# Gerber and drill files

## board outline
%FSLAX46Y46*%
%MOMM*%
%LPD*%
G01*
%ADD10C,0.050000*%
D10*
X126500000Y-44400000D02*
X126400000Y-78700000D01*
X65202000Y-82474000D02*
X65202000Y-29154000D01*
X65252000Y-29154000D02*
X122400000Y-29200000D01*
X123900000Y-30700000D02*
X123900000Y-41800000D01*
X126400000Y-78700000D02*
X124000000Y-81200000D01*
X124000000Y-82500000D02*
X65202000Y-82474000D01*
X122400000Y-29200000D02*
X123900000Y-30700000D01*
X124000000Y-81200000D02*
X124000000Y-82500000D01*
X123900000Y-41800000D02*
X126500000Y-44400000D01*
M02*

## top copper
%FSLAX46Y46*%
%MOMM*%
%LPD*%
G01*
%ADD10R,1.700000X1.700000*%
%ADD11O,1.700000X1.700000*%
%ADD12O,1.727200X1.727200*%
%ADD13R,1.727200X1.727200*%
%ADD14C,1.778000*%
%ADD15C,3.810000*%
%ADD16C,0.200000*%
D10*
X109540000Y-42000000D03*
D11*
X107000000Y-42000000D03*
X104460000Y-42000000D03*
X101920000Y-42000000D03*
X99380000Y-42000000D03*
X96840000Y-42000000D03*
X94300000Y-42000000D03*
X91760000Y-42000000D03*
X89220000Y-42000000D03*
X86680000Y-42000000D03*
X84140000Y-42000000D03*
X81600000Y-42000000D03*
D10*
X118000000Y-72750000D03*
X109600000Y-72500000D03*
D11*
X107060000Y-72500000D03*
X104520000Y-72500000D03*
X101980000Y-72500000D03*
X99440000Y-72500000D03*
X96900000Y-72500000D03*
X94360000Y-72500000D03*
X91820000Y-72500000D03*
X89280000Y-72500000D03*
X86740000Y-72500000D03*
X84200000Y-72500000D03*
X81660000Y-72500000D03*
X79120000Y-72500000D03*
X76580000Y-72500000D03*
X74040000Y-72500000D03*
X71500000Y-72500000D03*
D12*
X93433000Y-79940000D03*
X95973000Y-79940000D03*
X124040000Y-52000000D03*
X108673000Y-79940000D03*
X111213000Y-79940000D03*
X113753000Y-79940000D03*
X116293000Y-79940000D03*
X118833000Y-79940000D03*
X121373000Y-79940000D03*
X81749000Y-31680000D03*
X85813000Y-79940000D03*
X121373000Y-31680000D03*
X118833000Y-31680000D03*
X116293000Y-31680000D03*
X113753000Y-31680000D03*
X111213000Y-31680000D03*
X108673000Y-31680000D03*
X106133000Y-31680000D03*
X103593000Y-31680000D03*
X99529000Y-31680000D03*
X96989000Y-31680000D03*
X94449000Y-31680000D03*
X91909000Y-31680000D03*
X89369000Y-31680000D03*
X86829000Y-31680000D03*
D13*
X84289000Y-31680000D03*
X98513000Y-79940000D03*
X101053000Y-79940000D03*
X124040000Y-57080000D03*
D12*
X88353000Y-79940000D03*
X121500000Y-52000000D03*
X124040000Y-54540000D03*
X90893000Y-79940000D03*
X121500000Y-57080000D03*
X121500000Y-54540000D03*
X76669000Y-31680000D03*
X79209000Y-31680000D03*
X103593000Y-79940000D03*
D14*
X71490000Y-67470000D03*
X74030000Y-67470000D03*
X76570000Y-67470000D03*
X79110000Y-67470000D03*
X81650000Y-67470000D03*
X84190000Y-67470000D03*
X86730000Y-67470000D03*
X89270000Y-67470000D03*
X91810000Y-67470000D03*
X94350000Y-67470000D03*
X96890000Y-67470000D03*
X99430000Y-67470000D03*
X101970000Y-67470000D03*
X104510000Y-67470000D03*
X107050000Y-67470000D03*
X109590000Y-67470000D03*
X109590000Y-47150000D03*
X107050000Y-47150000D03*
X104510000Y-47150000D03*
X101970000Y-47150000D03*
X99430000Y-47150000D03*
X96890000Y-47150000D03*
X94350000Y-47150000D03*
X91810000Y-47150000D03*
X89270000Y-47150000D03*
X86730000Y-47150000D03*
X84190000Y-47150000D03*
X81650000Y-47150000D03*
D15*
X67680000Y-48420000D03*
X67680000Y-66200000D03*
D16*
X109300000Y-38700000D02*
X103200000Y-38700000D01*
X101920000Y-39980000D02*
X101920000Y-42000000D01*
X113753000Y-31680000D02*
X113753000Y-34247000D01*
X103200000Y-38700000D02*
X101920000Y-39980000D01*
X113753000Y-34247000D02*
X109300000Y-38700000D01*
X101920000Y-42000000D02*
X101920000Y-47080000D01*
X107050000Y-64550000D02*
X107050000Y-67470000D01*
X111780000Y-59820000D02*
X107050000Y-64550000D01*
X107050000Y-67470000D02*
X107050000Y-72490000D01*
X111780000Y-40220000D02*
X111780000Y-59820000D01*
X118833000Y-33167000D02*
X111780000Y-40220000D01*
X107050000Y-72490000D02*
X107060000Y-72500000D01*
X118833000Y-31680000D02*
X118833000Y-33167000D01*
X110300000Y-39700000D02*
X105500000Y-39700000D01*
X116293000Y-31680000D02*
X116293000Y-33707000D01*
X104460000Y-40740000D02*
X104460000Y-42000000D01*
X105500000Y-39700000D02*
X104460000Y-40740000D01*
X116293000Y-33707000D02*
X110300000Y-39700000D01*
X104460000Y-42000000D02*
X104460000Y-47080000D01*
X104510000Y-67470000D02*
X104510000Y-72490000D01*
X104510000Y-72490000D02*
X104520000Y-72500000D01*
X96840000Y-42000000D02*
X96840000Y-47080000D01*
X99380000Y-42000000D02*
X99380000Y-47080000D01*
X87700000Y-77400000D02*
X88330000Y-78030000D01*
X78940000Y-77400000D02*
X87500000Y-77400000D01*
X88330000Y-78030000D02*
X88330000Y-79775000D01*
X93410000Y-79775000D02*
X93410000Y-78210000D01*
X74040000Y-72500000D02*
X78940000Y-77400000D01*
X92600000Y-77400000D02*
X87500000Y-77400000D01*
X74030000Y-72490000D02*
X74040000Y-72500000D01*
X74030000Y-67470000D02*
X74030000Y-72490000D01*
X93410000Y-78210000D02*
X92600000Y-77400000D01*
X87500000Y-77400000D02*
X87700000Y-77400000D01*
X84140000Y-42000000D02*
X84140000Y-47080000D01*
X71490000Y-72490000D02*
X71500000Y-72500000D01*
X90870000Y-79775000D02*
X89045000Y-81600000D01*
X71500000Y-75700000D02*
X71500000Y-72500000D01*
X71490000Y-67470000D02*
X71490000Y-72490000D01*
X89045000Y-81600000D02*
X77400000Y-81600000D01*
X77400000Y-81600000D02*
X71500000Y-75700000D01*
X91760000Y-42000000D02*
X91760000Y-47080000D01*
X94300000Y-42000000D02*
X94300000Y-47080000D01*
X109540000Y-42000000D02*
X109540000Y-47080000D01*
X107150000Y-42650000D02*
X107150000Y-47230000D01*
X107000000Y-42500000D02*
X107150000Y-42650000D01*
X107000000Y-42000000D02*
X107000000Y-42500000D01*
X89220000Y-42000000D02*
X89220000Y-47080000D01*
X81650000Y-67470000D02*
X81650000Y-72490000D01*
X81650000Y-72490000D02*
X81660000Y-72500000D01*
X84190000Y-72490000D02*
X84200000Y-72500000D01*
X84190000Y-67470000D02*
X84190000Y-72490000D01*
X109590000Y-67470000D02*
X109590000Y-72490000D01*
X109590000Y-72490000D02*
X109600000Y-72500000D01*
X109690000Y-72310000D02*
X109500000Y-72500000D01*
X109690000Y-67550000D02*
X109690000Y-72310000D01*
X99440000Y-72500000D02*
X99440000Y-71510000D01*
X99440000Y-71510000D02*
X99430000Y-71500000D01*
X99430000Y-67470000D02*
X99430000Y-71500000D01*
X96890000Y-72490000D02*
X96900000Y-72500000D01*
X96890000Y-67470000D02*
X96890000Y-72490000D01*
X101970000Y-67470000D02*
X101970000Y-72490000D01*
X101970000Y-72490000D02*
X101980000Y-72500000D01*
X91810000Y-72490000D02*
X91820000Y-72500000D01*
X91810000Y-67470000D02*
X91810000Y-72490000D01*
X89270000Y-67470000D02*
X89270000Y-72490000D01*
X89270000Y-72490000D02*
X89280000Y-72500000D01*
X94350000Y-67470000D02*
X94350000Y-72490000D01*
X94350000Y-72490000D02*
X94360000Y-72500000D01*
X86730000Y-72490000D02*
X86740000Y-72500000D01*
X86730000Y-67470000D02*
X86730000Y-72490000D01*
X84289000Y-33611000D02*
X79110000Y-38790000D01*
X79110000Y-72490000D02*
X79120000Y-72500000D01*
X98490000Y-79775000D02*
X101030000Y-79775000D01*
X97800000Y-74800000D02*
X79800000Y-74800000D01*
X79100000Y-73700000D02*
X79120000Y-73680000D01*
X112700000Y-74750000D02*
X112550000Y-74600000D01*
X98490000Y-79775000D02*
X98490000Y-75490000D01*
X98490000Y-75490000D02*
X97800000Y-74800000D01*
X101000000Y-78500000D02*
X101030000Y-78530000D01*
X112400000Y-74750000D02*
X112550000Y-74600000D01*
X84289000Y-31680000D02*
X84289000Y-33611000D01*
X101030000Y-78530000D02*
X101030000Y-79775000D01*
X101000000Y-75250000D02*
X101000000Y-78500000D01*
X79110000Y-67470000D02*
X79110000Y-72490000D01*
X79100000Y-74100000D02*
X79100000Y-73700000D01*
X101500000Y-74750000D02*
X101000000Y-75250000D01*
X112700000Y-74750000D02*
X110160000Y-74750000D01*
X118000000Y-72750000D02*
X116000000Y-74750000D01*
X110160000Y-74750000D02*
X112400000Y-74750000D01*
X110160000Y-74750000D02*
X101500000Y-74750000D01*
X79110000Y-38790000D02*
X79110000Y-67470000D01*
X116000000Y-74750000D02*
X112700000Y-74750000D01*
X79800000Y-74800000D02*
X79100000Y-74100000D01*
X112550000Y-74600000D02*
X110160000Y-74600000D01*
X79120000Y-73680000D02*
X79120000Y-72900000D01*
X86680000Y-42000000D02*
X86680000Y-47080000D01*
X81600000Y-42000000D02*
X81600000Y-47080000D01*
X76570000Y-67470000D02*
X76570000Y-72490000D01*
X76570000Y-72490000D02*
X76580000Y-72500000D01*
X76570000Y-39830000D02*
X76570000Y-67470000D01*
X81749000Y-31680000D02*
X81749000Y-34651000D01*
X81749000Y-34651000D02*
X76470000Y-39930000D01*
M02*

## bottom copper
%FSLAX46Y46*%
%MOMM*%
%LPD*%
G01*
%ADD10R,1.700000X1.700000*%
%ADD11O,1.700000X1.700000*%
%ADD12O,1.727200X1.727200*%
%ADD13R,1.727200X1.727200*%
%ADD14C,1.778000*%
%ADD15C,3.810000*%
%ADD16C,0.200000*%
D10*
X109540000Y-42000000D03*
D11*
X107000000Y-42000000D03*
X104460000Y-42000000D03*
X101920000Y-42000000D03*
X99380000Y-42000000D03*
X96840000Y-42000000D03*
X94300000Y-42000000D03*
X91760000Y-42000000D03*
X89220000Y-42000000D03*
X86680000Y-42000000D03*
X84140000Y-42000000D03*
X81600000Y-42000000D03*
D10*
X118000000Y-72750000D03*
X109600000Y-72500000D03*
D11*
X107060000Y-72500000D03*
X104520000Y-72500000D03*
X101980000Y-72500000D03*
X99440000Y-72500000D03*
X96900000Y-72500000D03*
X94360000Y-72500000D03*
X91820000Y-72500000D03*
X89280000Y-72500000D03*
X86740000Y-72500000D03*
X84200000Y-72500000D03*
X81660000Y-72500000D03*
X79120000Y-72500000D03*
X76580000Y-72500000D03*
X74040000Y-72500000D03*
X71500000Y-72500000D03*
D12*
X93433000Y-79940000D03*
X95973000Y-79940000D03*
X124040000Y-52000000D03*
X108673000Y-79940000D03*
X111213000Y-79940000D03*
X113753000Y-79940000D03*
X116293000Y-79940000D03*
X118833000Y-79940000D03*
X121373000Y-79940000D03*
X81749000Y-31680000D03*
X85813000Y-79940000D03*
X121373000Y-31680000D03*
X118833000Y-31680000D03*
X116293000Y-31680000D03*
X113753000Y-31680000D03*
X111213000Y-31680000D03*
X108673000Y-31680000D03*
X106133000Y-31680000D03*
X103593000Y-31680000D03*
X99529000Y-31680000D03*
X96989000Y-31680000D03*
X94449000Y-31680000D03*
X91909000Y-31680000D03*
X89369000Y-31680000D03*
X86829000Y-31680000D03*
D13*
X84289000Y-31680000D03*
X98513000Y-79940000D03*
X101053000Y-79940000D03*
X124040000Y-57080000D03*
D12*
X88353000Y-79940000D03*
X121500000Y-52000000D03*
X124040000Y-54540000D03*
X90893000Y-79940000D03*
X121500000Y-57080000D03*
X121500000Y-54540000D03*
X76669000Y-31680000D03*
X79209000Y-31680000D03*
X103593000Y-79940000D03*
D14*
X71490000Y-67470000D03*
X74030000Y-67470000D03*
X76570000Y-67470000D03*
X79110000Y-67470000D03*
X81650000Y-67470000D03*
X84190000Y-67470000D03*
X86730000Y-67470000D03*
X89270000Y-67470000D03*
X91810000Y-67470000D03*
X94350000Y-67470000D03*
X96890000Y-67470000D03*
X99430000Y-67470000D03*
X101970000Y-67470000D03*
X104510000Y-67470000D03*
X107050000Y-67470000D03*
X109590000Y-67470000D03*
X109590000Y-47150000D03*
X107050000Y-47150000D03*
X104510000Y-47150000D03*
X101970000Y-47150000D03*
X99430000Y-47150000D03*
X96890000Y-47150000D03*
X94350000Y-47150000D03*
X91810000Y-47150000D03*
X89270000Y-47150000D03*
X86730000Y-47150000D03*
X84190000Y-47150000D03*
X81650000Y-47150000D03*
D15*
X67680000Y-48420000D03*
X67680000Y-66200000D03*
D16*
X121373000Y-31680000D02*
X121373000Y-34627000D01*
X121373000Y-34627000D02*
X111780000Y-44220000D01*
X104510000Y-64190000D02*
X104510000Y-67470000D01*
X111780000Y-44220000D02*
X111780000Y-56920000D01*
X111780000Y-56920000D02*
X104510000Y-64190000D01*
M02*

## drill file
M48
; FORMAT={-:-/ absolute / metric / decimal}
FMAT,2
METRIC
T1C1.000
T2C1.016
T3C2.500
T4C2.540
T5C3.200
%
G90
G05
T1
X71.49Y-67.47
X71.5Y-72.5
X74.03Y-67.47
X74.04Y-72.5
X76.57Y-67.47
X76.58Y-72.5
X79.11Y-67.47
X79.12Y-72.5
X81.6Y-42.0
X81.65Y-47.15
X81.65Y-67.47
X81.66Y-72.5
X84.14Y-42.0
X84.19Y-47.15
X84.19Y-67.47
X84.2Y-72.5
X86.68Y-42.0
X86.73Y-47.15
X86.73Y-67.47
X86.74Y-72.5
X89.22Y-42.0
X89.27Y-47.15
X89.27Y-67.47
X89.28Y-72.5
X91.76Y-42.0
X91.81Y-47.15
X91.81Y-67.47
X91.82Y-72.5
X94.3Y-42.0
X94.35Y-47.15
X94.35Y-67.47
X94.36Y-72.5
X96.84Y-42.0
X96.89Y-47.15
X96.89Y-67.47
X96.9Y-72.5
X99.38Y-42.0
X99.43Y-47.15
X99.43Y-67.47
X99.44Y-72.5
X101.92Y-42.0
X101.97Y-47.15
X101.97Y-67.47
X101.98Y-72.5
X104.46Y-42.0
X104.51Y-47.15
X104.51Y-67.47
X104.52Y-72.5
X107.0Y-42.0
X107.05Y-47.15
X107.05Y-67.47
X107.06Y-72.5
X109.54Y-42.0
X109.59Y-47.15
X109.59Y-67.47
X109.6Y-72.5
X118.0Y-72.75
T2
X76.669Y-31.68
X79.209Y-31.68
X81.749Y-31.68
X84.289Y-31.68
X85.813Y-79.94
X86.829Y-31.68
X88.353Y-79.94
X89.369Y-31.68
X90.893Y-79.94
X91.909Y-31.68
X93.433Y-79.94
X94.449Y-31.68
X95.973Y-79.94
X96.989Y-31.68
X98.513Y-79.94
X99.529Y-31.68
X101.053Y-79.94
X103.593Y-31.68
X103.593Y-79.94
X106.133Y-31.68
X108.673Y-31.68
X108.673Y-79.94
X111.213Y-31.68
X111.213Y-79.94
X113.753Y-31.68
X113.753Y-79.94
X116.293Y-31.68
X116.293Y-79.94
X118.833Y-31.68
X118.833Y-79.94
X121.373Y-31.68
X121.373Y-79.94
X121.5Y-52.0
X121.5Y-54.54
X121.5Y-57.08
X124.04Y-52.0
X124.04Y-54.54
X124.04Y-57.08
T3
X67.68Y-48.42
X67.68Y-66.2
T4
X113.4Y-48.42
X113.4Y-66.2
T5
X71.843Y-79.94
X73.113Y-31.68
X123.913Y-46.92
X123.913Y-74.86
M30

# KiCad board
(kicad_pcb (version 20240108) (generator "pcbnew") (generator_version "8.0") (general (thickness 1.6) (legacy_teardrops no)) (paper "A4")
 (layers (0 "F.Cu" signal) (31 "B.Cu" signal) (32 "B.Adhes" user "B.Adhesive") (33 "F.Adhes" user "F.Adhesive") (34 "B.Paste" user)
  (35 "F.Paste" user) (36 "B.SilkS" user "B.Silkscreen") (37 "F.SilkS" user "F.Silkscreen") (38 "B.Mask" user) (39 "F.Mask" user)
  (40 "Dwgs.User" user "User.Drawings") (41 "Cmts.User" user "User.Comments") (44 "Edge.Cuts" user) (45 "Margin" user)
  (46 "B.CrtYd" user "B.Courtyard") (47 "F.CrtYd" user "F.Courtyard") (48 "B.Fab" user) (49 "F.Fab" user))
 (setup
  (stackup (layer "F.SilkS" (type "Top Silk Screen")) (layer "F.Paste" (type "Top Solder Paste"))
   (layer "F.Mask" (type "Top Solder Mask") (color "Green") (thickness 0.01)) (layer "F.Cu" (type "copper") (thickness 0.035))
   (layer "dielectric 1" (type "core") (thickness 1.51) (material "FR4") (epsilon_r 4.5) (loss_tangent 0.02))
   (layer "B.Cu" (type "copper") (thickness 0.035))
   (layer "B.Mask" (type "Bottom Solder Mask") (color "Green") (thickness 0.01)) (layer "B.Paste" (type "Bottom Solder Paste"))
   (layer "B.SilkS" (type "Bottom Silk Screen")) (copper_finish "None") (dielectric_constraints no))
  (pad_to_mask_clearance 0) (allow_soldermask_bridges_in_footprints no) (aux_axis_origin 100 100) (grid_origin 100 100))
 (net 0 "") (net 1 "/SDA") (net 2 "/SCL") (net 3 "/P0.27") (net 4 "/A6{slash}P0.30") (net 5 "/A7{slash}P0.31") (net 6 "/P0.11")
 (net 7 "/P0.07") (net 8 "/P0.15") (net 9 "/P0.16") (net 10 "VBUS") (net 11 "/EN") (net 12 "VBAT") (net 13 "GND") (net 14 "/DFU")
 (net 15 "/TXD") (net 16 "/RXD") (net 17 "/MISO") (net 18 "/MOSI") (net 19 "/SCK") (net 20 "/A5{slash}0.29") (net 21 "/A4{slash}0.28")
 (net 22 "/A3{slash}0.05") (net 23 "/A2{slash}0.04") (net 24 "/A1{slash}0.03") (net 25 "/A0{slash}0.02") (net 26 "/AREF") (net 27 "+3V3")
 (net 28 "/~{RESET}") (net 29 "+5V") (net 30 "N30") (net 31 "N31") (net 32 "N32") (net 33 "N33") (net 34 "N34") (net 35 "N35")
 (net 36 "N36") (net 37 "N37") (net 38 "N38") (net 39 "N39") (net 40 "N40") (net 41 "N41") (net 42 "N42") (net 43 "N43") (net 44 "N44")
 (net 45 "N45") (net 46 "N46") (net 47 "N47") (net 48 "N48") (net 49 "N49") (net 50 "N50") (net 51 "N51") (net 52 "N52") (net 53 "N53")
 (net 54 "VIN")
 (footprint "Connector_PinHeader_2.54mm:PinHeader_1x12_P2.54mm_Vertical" (layer "F.Cu") (at 109.54 42 -90)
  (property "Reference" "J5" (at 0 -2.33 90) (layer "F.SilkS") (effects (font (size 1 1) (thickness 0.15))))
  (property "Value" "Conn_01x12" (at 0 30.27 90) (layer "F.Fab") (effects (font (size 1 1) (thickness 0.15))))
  (pad "1" thru_hole rect (at 0 0 270) (size 1.7 1.7) (drill 1) (layers "*.Cu" "*.Mask") (remove_unused_layers no) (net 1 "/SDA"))
  (pad "2" thru_hole oval (at 0 2.54 270) (size 1.7 1.7) (drill 1) (layers "*.Cu" "*.Mask") (remove_unused_layers no) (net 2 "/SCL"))
  (pad "3" thru_hole oval (at 0 5.08 270) (size 1.7 1.7) (drill 1) (layers "*.Cu" "*.Mask") (remove_unused_layers no) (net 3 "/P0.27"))
  (pad "4" thru_hole oval (at 0 7.62 270) (size 1.7 1.7) (drill 1) (layers "*.Cu" "*.Mask") (remove_unused_layers no)
   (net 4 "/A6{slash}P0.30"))
  (pad "5" thru_hole oval (at 0 10.16 270) (size 1.7 1.7) (drill 1) (layers "*.Cu" "*.Mask") (remove_unused_layers no)
   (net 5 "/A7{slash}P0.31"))
  (pad "6" thru_hole oval (at 0 12.7 270) (size 1.7 1.7) (drill 1) (layers "*.Cu" "*.Mask") (remove_unused_layers no) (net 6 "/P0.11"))
  (pad "7" thru_hole oval (at 0 15.24 270) (size 1.7 1.7) (drill 1) (layers "*.Cu" "*.Mask") (remove_unused_layers no) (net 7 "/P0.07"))
  (pad "8" thru_hole oval (at 0 17.78 270) (size 1.7 1.7) (drill 1) (layers "*.Cu" "*.Mask") (remove_unused_layers no) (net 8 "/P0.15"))
  (pad "9" thru_hole oval (at 0 20.32 270) (size 1.7 1.7) (drill 1) (layers "*.Cu" "*.Mask") (remove_unused_layers no) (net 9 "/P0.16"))
  (pad "10" thru_hole oval (at 0 22.86 270) (size 1.7 1.7) (drill 1) (layers "*.Cu" "*.Mask") (remove_unused_layers no) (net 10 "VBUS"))
  (pad "11" thru_hole oval (at 0 25.4 270) (size 1.7 1.7) (drill 1) (layers "*.Cu" "*.Mask") (remove_unused_layers no) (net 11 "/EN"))
  (pad "12" thru_hole oval (at 0 27.94 270) (size 1.7 1.7) (drill 1) (layers "*.Cu" "*.Mask") (remove_unused_layers no) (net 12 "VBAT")))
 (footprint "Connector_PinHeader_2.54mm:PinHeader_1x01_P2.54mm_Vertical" (layer "F.Cu") (at 118 72.75)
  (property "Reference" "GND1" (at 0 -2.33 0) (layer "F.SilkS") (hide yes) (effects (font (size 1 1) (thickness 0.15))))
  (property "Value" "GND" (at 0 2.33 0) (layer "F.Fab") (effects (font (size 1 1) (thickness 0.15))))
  (pad "1" thru_hole rect (at 0 0) (size 1.7 1.7) (drill 1) (layers "*.Cu" "*.Mask") (remove_unused_layers no) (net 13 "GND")))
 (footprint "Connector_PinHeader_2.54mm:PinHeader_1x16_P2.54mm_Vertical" (layer "F.Cu") (at 109.6 72.5 -90)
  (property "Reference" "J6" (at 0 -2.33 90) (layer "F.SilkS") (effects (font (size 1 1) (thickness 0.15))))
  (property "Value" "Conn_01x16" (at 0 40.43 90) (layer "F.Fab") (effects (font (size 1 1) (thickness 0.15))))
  (pad "1" thru_hole rect (at 0 0 270) (size 1.7 1.7) (drill 1) (layers "*.Cu" "*.Mask") (remove_unused_layers no) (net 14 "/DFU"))
  (pad "2" thru_hole oval (at 0 2.54 270) (size 1.7 1.7) (drill 1) (layers "*.Cu" "*.Mask") (remove_unused_layers no) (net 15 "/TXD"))
  (pad "3" thru_hole oval (at 0 5.08 270) (size 1.7 1.7) (drill 1) (layers "*.Cu" "*.Mask") (remove_unused_layers no) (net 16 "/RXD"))
  (pad "4" thru_hole oval (at 0 7.62 270) (size 1.7 1.7) (drill 1) (layers "*.Cu" "*.Mask") (remove_unused_layers no) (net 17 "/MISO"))
  (pad "5" thru_hole oval (at 0 10.16 270) (size 1.7 1.7) (drill 1) (layers "*.Cu" "*.Mask") (remove_unused_layers no) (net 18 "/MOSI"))
  (pad "6" thru_hole oval (at 0 12.7 270) (size 1.7 1.7) (drill 1) (layers "*.Cu" "*.Mask") (remove_unused_layers no) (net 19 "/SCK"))
  (pad "7" thru_hole oval (at 0 15.24 270) (size 1.7 1.7) (drill 1) (layers "*.Cu" "*.Mask") (remove_unused_layers no)
   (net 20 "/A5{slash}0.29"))
  (pad "8" thru_hole oval (at 0 17.78 270) (size 1.7 1.7) (drill 1) (layers "*.Cu" "*.Mask") (remove_unused_layers no)
   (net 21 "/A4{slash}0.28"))
  (pad "9" thru_hole oval (at 0 20.32 270) (size 1.7 1.7) (drill 1) (layers "*.Cu" "*.Mask") (remove_unused_layers no)
   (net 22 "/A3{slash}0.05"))
  (pad "10" thru_hole oval (at 0 22.86 270) (size 1.7 1.7) (drill 1) (layers "*.Cu" "*.Mask") (remove_unused_layers no)
   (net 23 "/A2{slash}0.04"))
  (pad "11" thru_hole oval (at 0 25.4 270) (size 1.7 1.7) (drill 1) (layers "*.Cu" "*.Mask") (remove_unused_layers no)
   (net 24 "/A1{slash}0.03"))
  (pad "12" thru_hole oval (at 0 27.94 270) (size 1.7 1.7) (drill 1) (layers "*.Cu" "*.Mask") (remove_unused_layers no)
   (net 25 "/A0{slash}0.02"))
  (pad "13" thru_hole oval (at 0 30.48 270) (size 1.7 1.7) (drill 1) (layers "*.Cu" "*.Mask") (remove_unused_layers no) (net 13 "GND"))
  (pad "14" thru_hole oval (at 0 33.02 270) (size 1.7 1.7) (drill 1) (layers "*.Cu" "*.Mask") (remove_unused_layers no) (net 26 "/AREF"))
  (pad "15" thru_hole oval (at 0 35.56 270) (size 1.7 1.7) (drill 1) (layers "*.Cu" "*.Mask") (remove_unused_layers no) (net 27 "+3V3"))
  (pad "16" thru_hole oval (at 0 38.1 270) (size 1.7 1.7) (drill 1) (layers "*.Cu" "*.Mask") (remove_unused_layers no) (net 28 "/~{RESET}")))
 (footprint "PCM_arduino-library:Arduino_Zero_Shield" (layer "F.Cu") (at 57.873 82.48)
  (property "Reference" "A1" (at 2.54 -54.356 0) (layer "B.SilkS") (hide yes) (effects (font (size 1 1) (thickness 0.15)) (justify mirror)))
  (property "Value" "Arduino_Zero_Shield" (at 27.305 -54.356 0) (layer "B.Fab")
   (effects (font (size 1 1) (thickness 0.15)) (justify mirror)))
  (pad "" np_thru_hole circle (at 13.97 -2.54) (size 3.2 3.2) (drill 3.2) (layers "*.Cu" "*.Mask"))
  (pad "" np_thru_hole circle (at 15.24 -50.8) (size 3.2 3.2) (drill 3.2) (layers "*.Cu" "*.Mask"))
  (pad "" np_thru_hole circle (at 66.04 -35.56) (size 3.2 3.2) (drill 3.2) (layers "*.Cu" "*.Mask"))
  (pad "" np_thru_hole circle (at 66.04 -7.62) (size 3.2 3.2) (drill 3.2) (layers "*.Cu" "*.Mask"))
  (pad "3V3" thru_hole oval (at 35.56 -2.54) (size 1.7272 1.7272) (drill 1.016) (layers "*.Cu" "*.Mask") (remove_unused_layers no)
   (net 27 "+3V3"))
  (pad "5V1" thru_hole oval (at 38.1 -2.54) (size 1.7272 1.7272) (drill 1.016) (layers "*.Cu" "*.Mask") (remove_unused_layers no)
   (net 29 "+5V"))
  (pad "5V2" thru_hole oval (at 66.167 -30.48) (size 1.7272 1.7272) (drill 1.016) (layers "*.Cu" "*.Mask") (remove_unused_layers no)
   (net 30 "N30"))
  (pad "A0" thru_hole oval (at 50.8 -2.54) (size 1.7272 1.7272) (drill 1.016) (layers "*.Cu" "*.Mask") (remove_unused_layers no)
   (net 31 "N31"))
  (pad "A1" thru_hole oval (at 53.34 -2.54) (size 1.7272 1.7272) (drill 1.016) (layers "*.Cu" "*.Mask") (remove_unused_layers no)
   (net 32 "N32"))
  (pad "A2" thru_hole oval (at 55.88 -2.54) (size 1.7272 1.7272) (drill 1.016) (layers "*.Cu" "*.Mask") (remove_unused_layers no)
   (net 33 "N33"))
  (pad "A3" thru_hole oval (at 58.42 -2.54) (size 1.7272 1.7272) (drill 1.016) (layers "*.Cu" "*.Mask") (remove_unused_layers no)
   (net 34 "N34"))
  (pad "A4" thru_hole oval (at 60.96 -2.54) (size 1.7272 1.7272) (drill 1.016) (layers "*.Cu" "*.Mask") (remove_unused_layers no)
   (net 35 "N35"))
  (pad "A5" thru_hole oval (at 63.5 -2.54) (size 1.7272 1.7272) (drill 1.016) (layers "*.Cu" "*.Mask") (remove_unused_layers no)
   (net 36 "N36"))
  (pad "AREF" thru_hole oval (at 23.876 -50.8) (size 1.7272 1.7272) (drill 1.016) (layers "*.Cu" "*.Mask") (remove_unused_layers no)
   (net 26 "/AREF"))
  (pad "ATN" thru_hole oval (at 27.94 -2.54) (size 1.7272 1.7272) (drill 1.016) (layers "*.Cu" "*.Mask") (remove_unused_layers no)
   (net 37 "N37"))
  (pad "D0" thru_hole oval (at 63.5 -50.8) (size 1.7272 1.7272) (drill 1.016) (layers "*.Cu" "*.Mask") (remove_unused_layers no)
   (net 16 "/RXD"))
  (pad "D1" thru_hole oval (at 60.96 -50.8) (size 1.7272 1.7272) (drill 1.016) (layers "*.Cu" "*.Mask") (remove_unused_layers no)
   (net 15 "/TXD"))
  (pad "D2" thru_hole oval (at 58.42 -50.8) (size 1.7272 1.7272) (drill 1.016) (layers "*.Cu" "*.Mask") (remove_unused_layers no)
   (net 3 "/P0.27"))
  (pad "D3" thru_hole oval (at 55.88 -50.8) (size 1.7272 1.7272) (drill 1.016) (layers "*.Cu" "*.Mask") (remove_unused_layers no)
   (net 4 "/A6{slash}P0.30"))
  (pad "D4" thru_hole oval (at 53.34 -50.8) (size 1.7272 1.7272) (drill 1.016) (layers "*.Cu" "*.Mask") (remove_unused_layers no)
   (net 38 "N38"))
  (pad "D5" thru_hole oval (at 50.8 -50.8) (size 1.7272 1.7272) (drill 1.016) (layers "*.Cu" "*.Mask") (remove_unused_layers no)
   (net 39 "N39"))
  (pad "D6" thru_hole oval (at 48.26 -50.8) (size 1.7272 1.7272) (drill 1.016) (layers "*.Cu" "*.Mask") (remove_unused_layers no)
   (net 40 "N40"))
  (pad "D7" thru_hole oval (at 45.72 -50.8) (size 1.7272 1.7272) (drill 1.016) (layers "*.Cu" "*.Mask") (remove_unused_layers no)
   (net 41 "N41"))
  (pad "D8" thru_hole oval (at 41.656 -50.8) (size 1.7272 1.7272) (drill 1.016) (layers "*.Cu" "*.Mask") (remove_unused_layers no)
   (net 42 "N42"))
  (pad "D9" thru_hole oval (at 39.116 -50.8) (size 1.7272 1.7272) (drill 1.016) (layers "*.Cu" "*.Mask") (remove_unused_layers no)
   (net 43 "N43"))
  (pad "D10" thru_hole oval (at 36.576 -50.8) (size 1.7272 1.7272) (drill 1.016) (layers "*.Cu" "*.Mask") (remove_unused_layers no)
   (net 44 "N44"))
  (pad "D11" thru_hole oval (at 34.036 -50.8) (size 1.7272 1.7272) (drill 1.016) (layers "*.Cu" "*.Mask") (remove_unused_layers no)
   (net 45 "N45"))
  (pad "D12" thru_hole oval (at 31.496 -50.8) (size 1.7272 1.7272) (drill 1.016) (layers "*.Cu" "*.Mask") (remove_unused_layers no)
   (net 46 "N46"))
  (pad "D13" thru_hole oval (at 28.956 -50.8) (size 1.7272 1.7272) (drill 1.016) (layers "*.Cu" "*.Mask") (remove_unused_layers no)
   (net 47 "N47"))
  (pad "GND1" thru_hole rect (at 26.416 -50.8) (size 1.7272 1.7272) (drill 1.016) (layers "*.Cu" "*.Mask") (remove_unused_layers no)
   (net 13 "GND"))
  (pad "GND2" thru_hole rect (at 40.64 -2.54) (size 1.7272 1.7272) (drill 1.016) (layers "*.Cu" "*.Mask") (remove_unused_layers no)
   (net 13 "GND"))
  (pad "GND3" thru_hole rect (at 43.18 -2.54) (size 1.7272 1.7272) (drill 1.016) (layers "*.Cu" "*.Mask") (remove_unused_layers no)
   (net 13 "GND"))
  (pad "GND4" thru_hole rect (at 66.167 -25.4) (size 1.7272 1.7272) (drill 1.016) (layers "*.Cu" "*.Mask") (remove_unused_layers no)
   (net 13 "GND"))
  (pad "IORF" thru_hole oval (at 30.48 -2.54) (size 1.7272 1.7272) (drill 1.016) (layers "*.Cu" "*.Mask") (remove_unused_layers no)
   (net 27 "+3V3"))
  (pad "MISO" thru_hole oval (at 63.627 -30.48) (size 1.7272 1.7272) (drill 1.016) (layers "*.Cu" "*.Mask") (remove_unused_layers no)
   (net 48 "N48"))
  (pad "MOSI" thru_hole oval (at 66.167 -27.94) (size 1.7272 1.7272) (drill 1.016) (layers "*.Cu" "*.Mask") (remove_unused_layers no)
   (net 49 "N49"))
  (pad "RST1" thru_hole oval (at 33.02 -2.54) (size 1.7272 1.7272) (drill 1.016) (layers "*.Cu" "*.Mask") (remove_unused_layers no)
   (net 28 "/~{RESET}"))
  (pad "RST2" thru_hole oval (at 63.627 -25.4) (size 1.7272 1.7272) (drill 1.016) (layers "*.Cu" "*.Mask") (remove_unused_layers no)
   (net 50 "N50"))
  (pad "SCK" thru_hole oval (at 63.627 -27.94) (size 1.7272 1.7272) (drill 1.016) (layers "*.Cu" "*.Mask") (remove_unused_layers no)
   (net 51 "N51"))
  (pad "SCL" thru_hole oval (at 18.796 -50.8) (size 1.7272 1.7272) (drill 1.016) (layers "*.Cu" "*.Mask") (remove_unused_layers no)
   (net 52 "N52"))
  (pad "SDA" thru_hole oval (at 21.336 -50.8) (size 1.7272 1.7272) (drill 1.016) (layers "*.Cu" "*.Mask") (remove_unused_layers no)
   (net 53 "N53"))
  (pad "VIN" thru_hole oval (at 45.72 -2.54) (size 1.7272 1.7272) (drill 1.016) (layers "*.Cu" "*.Mask") (remove_unused_layers no)
   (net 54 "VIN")))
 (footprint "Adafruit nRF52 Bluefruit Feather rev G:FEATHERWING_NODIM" (layer "F.Cu") (at 65.14 68.74)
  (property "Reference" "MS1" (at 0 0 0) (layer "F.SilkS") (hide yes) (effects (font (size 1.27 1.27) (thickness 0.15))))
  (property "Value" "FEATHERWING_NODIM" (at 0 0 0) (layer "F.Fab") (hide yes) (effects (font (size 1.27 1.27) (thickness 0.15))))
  (pad "" np_thru_hole circle (at 48.26 -20.32) (size 2.54 2.54) (drill 2.54) (layers "*.Cu" "*.Mask"))
  (pad "" np_thru_hole circle (at 48.26 -2.54) (size 2.54 2.54) (drill 2.54) (layers "*.Cu" "*.Mask"))
  (pad "1" thru_hole circle (at 6.35 -1.27) (size 1.778 1.778) (drill 1) (layers "*.Cu" "*.Mask") (remove_unused_layers no)
   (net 28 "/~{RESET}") (solder_mask_margin 0.0508) (thermal_bridge_angle 0))
  (pad "2" thru_hole circle (at 8.89 -1.27) (size 1.778 1.778) (drill 1) (layers "*.Cu" "*.Mask") (remove_unused_layers no) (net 27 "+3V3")
   (solder_mask_margin 0.0508) (thermal_bridge_angle 0))
  (pad "3" thru_hole circle (at 11.43 -1.27) (size 1.778 1.778) (drill 1) (layers "*.Cu" "*.Mask") (remove_unused_layers no)
   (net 26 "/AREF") (solder_mask_margin 0.0508) (thermal_bridge_angle 0))
  (pad "4" thru_hole circle (at 13.97 -1.27) (size 1.778 1.778) (drill 1) (layers "*.Cu" "*.Mask") (remove_unused_layers no) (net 13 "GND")
   (solder_mask_margin 0.0508) (thermal_bridge_angle 0))
  (pad "5" thru_hole circle (at 16.51 -1.27) (size 1.778 1.778) (drill 1) (layers "*.Cu" "*.Mask") (remove_unused_layers no)
   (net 25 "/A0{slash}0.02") (solder_mask_margin 0.0508) (thermal_bridge_angle 0))
  (pad "6" thru_hole circle (at 19.05 -1.27) (size 1.778 1.778) (drill 1) (layers "*.Cu" "*.Mask") (remove_unused_layers no)
   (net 24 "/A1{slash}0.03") (solder_mask_margin 0.0508) (thermal_bridge_angle 0))
  (pad "7" thru_hole circle (at 21.59 -1.27) (size 1.778 1.778) (drill 1) (layers "*.Cu" "*.Mask") (remove_unused_layers no)
   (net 23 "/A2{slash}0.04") (solder_mask_margin 0.0508) (thermal_bridge_angle 0))
  (pad "8" thru_hole circle (at 24.13 -1.27) (size 1.778 1.778) (drill 1) (layers "*.Cu" "*.Mask") (remove_unused_layers no)
   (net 22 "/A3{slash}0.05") (solder_mask_margin 0.0508) (thermal_bridge_angle 0))
  (pad "9" thru_hole circle (at 26.67 -1.27) (size 1.778 1.778) (drill 1) (layers "*.Cu" "*.Mask") (remove_unused_layers no)
   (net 21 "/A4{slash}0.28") (solder_mask_margin 0.0508) (thermal_bridge_angle 0))
  (pad "10" thru_hole circle (at 29.21 -1.27) (size 1.778 1.778) (drill 1) (layers "*.Cu" "*.Mask") (remove_unused_layers no)
   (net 20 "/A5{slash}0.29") (solder_mask_margin 0.0508) (thermal_bridge_angle 0))
  (pad "11" thru_hole circle (at 31.75 -1.27) (size 1.778 1.778) (drill 1) (layers "*.Cu" "*.Mask") (remove_unused_layers no)
   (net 19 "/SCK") (solder_mask_margin 0.0508) (thermal_bridge_angle 0))
  (pad "12" thru_hole circle (at 34.29 -1.27) (size 1.778 1.778) (drill 1) (layers "*.Cu" "*.Mask") (remove_unused_layers no)
   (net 18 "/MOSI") (solder_mask_margin 0.0508) (thermal_bridge_angle 0))
  (pad "13" thru_hole circle (at 36.83 -1.27) (size 1.778 1.778) (drill 1) (layers "*.Cu" "*.Mask") (remove_unused_layers no)
   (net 17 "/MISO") (solder_mask_margin 0.0508) (thermal_bridge_angle 0))
  (pad "14" thru_hole circle (at 39.37 -1.27) (size 1.778 1.778) (drill 1) (layers "*.Cu" "*.Mask") (remove_unused_layers no)
   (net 16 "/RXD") (solder_mask_margin 0.0508) (thermal_bridge_angle 0))
  (pad "15" thru_hole circle (at 41.91 -1.27) (size 1.778 1.778) (drill 1) (layers "*.Cu" "*.Mask") (remove_unused_layers no)
   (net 15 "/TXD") (solder_mask_margin 0.0508) (thermal_bridge_angle 0))
  (pad "16" thru_hole circle (at 44.45 -1.27) (size 1.778 1.778) (drill 1) (layers "*.Cu" "*.Mask") (remove_unused_layers no)
   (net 14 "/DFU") (solder_mask_margin 0.0508) (thermal_bridge_angle 0))
  (pad "17" thru_hole circle (at 44.45 -21.59) (size 1.778 1.778) (drill 1) (layers "*.Cu" "*.Mask") (remove_unused_layers no)
   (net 1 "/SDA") (solder_mask_margin 0.0508) (thermal_bridge_angle 0))
  (pad "18" thru_hole circle (at 41.91 -21.59) (size 1.778 1.778) (drill 1) (layers "*.Cu" "*.Mask") (remove_unused_layers no)
   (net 2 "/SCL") (solder_mask_margin 0.0508) (thermal_bridge_angle 0))
  (pad "19" thru_hole circle (at 39.37 -21.59) (size 1.778 1.778) (drill 1) (layers "*.Cu" "*.Mask") (remove_unused_layers no)
   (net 3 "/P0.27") (solder_mask_margin 0.0508) (thermal_bridge_angle 0))
  (pad "20" thru_hole circle (at 36.83 -21.59) (size 1.778 1.778) (drill 1) (layers "*.Cu" "*.Mask") (remove_unused_layers no)
   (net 4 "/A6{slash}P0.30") (solder_mask_margin 0.0508) (thermal_bridge_angle 0))
  (pad "21" thru_hole circle (at 34.29 -21.59) (size 1.778 1.778) (drill 1) (layers "*.Cu" "*.Mask") (remove_unused_layers no)
   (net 5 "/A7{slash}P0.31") (solder_mask_margin 0.0508) (thermal_bridge_angle 0))
  (pad "22" thru_hole circle (at 31.75 -21.59) (size 1.778 1.778) (drill 1) (layers "*.Cu" "*.Mask") (remove_unused_layers no)
   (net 6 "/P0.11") (solder_mask_margin 0.0508) (thermal_bridge_angle 0))
  (pad "23" thru_hole circle (at 29.21 -21.59) (size 1.778 1.778) (drill 1) (layers "*.Cu" "*.Mask") (remove_unused_layers no)
   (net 7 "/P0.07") (solder_mask_margin 0.0508) (thermal_bridge_angle 0))
  (pad "24" thru_hole circle (at 26.67 -21.59) (size 1.778 1.778) (drill 1) (layers "*.Cu" "*.Mask") (remove_unused_layers no)
   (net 8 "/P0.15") (solder_mask_margin 0.0508) (thermal_bridge_angle 0))
  (pad "25" thru_hole circle (at 24.13 -21.59) (size 1.778 1.778) (drill 1) (layers "*.Cu" "*.Mask") (remove_unused_layers no)
   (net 9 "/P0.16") (solder_mask_margin 0.0508) (thermal_bridge_angle 0))
  (pad "26" thru_hole circle (at 21.59 -21.59) (size 1.778 1.778) (drill 1) (layers "*.Cu" "*.Mask") (remove_unused_layers no)
   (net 10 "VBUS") (solder_mask_margin 0.0508) (thermal_bridge_angle 0))
  (pad "27" thru_hole circle (at 19.05 -21.59) (size 1.778 1.778) (drill 1) (layers "*.Cu" "*.Mask") (remove_unused_layers no)
   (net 11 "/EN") (solder_mask_margin 0.0508) (thermal_bridge_angle 0))
  (pad "28" thru_hole circle (at 16.51 -21.59) (size 1.778 1.778) (drill 1) (layers "*.Cu" "*.Mask") (remove_unused_layers no)
   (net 12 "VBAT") (solder_mask_margin 0.0508) (thermal_bridge_angle 0))
  (pad "P$1" thru_hole circle (at 2.54 -20.32) (size 3.81 3.81) (drill 2.5) (layers "*.Cu" "*.Mask") (remove_unused_layers no)
   (solder_mask_margin 0.0508) (thermal_bridge_angle 0))
  (pad "P$2" thru_hole circle (at 2.54 -2.54) (size 3.81 3.81) (drill 2.5) (layers "*.Cu" "*.Mask") (remove_unused_layers no)
   (solder_mask_margin 0.0508) (thermal_bridge_angle 0)))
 (gr_line (start 126.5 44.4) (end 126.4 78.7) (stroke (width 0.05) (type default)) (layer "Edge.Cuts"))
 (gr_line (start 65.202 82.474) (end 65.202 29.154) (stroke (width 0.05) (type default)) (layer "Edge.Cuts"))
 (gr_line (start 65.252 29.154) (end 122.4 29.2) (stroke (width 0.05) (type default)) (layer "Edge.Cuts"))
 (gr_line (start 123.9 30.7) (end 123.9 41.8) (stroke (width 0.05) (type default)) (layer "Edge.Cuts"))
 (gr_line (start 126.4 78.7) (end 124 81.2) (stroke (width 0.05) (type default)) (layer "Edge.Cuts"))
 (gr_line (start 124 82.5) (end 65.202 82.474) (stroke (width 0.05) (type default)) (layer "Edge.Cuts"))
 (gr_line (start 122.4 29.2) (end 123.9 30.7) (stroke (width 0.05) (type default)) (layer "Edge.Cuts"))
 (gr_line (start 124 81.2) (end 124 82.5) (stroke (width 0.05) (type default)) (layer "Edge.Cuts"))
 (gr_line (start 123.9 41.8) (end 126.5 44.4) (stroke (width 0.05) (type default)) (layer "Edge.Cuts"))
 (segment (start 109.3 38.7) (end 103.2 38.7) (width 0.2) (layer "F.Cu") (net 4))
 (segment (start 101.92 39.98) (end 101.92 42) (width 0.2) (layer "F.Cu") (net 4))
 (segment (start 113.753 31.68) (end 113.753 34.247) (width 0.2) (layer "F.Cu") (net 4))
 (segment (start 103.2 38.7) (end 101.92 39.98) (width 0.2) (layer "F.Cu") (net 4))
 (segment (start 113.753 34.247) (end 109.3 38.7) (width 0.2) (layer "F.Cu") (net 4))
 (segment (start 101.92 42) (end 101.92 47.08) (width 0.2) (layer "F.Cu") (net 4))
 (segment (start 107.05 64.55) (end 107.05 67.47) (width 0.2) (layer "F.Cu") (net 15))
 (segment (start 111.78 59.82) (end 107.05 64.55) (width 0.2) (layer "F.Cu") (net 15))
 (segment (start 107.05 67.47) (end 107.05 72.49) (width 0.2) (layer "F.Cu") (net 15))
 (segment (start 111.78 40.22) (end 111.78 59.82) (width 0.2) (layer "F.Cu") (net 15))
 (segment (start 118.833 33.167) (end 111.78 40.22) (width 0.2) (layer "F.Cu") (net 15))
 (segment (start 107.05 72.49) (end 107.06 72.5) (width 0.2) (layer "F.Cu") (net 15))
 (segment (start 118.833 31.68) (end 118.833 33.167) (width 0.2) (layer "F.Cu") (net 15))
 (segment (start 110.3 39.7) (end 105.5 39.7) (width 0.2) (layer "F.Cu") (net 3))
 (segment (start 116.293 31.68) (end 116.293 33.707) (width 0.2) (layer "F.Cu") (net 3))
 (segment (start 104.46 40.74) (end 104.46 42) (width 0.2) (layer "F.Cu") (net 3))
 (segment (start 105.5 39.7) (end 104.46 40.74) (width 0.2) (layer "F.Cu") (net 3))
 (segment (start 116.293 33.707) (end 110.3 39.7) (width 0.2) (layer "F.Cu") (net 3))
 (segment (start 104.46 42) (end 104.46 47.08) (width 0.2) (layer "F.Cu") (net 3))
 (segment (start 104.51 67.47) (end 104.51 72.49) (width 0.2) (layer "F.Cu") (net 16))
 (segment (start 104.51 72.49) (end 104.52 72.5) (width 0.2) (layer "F.Cu") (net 16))
 (segment (start 121.373 31.68) (end 121.373 34.627) (width 0.2) (layer "B.Cu") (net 16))
 (segment (start 121.373 34.627) (end 111.78 44.22) (width 0.2) (layer "B.Cu") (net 16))
 (segment (start 104.51 64.19) (end 104.51 67.47) (width 0.2) (layer "B.Cu") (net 16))
 (segment (start 111.78 44.22) (end 111.78 56.92) (width 0.2) (layer "B.Cu") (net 16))
 (segment (start 111.78 56.92) (end 104.51 64.19) (width 0.2) (layer "B.Cu") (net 16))
 (segment (start 96.84 42) (end 96.84 47.08) (width 0.2) (layer "F.Cu") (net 6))
 (segment (start 99.38 42) (end 99.38 47.08) (width 0.2) (layer "F.Cu") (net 5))
 (segment (start 87.7 77.4) (end 88.33 78.03) (width 0.2) (layer "F.Cu") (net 27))
 (segment (start 78.94 77.4) (end 87.5 77.4) (width 0.2) (layer "F.Cu") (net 27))
 (segment (start 88.33 78.03) (end 88.33 79.775) (width 0.2) (layer "F.Cu") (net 27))
 (segment (start 93.41 79.775) (end 93.41 78.21) (width 0.2) (layer "F.Cu") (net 27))
 (segment (start 74.04 72.5) (end 78.94 77.4) (width 0.2) (layer "F.Cu") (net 27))
 (segment (start 92.6 77.4) (end 87.5 77.4) (width 0.2) (layer "F.Cu") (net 27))
 (segment (start 74.03 72.49) (end 74.04 72.5) (width 0.2) (layer "F.Cu") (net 27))
 (segment (start 74.03 67.47) (end 74.03 72.49) (width 0.2) (layer "F.Cu") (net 27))
 (segment (start 93.41 78.21) (end 92.6 77.4) (width 0.2) (layer "F.Cu") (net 27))
 (segment (start 87.5 77.4) (end 87.7 77.4) (width 0.2) (layer "F.Cu") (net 27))
 (segment (start 84.14 42) (end 84.14 47.08) (width 0.2) (layer "F.Cu") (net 11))
 (segment (start 71.49 72.49) (end 71.5 72.5) (width 0.2) (layer "F.Cu") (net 28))
 (segment (start 90.87 79.775) (end 89.045 81.6) (width 0.2) (layer "F.Cu") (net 28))
 (segment (start 71.5 75.7) (end 71.5 72.5) (width 0.2) (layer "F.Cu") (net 28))
 (segment (start 71.49 67.47) (end 71.49 72.49) (width 0.2) (layer "F.Cu") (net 28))
 (segment (start 89.045 81.6) (end 77.4 81.6) (width 0.2) (layer "F.Cu") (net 28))
 (segment (start 77.4 81.6) (end 71.5 75.7) (width 0.2) (layer "F.Cu") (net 28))
 (segment (start 91.76 42) (end 91.76 47.08) (width 0.2) (layer "F.Cu") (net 8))
 (segment (start 94.3 42) (end 94.3 47.08) (width 0.2) (layer "F.Cu") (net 7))
 (segment (start 109.54 42) (end 109.54 47.08) (width 0.2) (layer "F.Cu") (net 1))
 (segment (start 107.15 42.65) (end 107.15 47.23) (width 0.2) (layer "F.Cu") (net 2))
 (segment (start 107 42.5) (end 107.15 42.65) (width 0.2) (layer "F.Cu") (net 2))
 (segment (start 107 42) (end 107 42.5) (width 0.2) (layer "F.Cu") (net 2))
 (segment (start 89.22 42) (end 89.22 47.08) (width 0.2) (layer "F.Cu") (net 9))
 (segment (start 81.65 67.47) (end 81.65 72.49) (width 0.2) (layer "F.Cu") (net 25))
 (segment (start 81.65 72.49) (end 81.66 72.5) (width 0.2) (layer "F.Cu") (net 25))
 (segment (start 84.19 72.49) (end 84.2 72.5) (width 0.2) (layer "F.Cu") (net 24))
 (segment (start 84.19 67.47) (end 84.19 72.49) (width 0.2) (layer "F.Cu") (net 24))
 (segment (start 109.59 67.47) (end 109.59 72.49) (width 0.2) (layer "F.Cu") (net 14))
 (segment (start 109.59 72.49) (end 109.6 72.5) (width 0.2) (layer "F.Cu") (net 14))
 (segment (start 109.69 72.31) (end 109.5 72.5) (width 0.2) (layer "F.Cu") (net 14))
 (segment (start 109.69 67.55) (end 109.69 72.31) (width 0.2) (layer "F.Cu") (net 14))
 (segment (start 99.44 72.5) (end 99.44 71.51) (width 0.2) (layer "F.Cu") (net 18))
 (segment (start 99.44 71.51) (end 99.43 71.5) (width 0.2) (layer "F.Cu") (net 18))
 (segment (start 99.43 67.47) (end 99.43 71.5) (width 0.2) (layer "F.Cu") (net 18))
 (segment (start 96.89 72.49) (end 96.9 72.5) (width 0.2) (layer "F.Cu") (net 19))
 (segment (start 96.89 67.47) (end 96.89 72.49) (width 0.2) (layer "F.Cu") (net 19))
 (segment (start 101.97 67.47) (end 101.97 72.49) (width 0.2) (layer "F.Cu") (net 17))
 (segment (start 101.97 72.49) (end 101.98 72.5) (width 0.2) (layer "F.Cu") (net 17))
 (segment (start 91.81 72.49) (end 91.82 72.5) (width 0.2) (layer "F.Cu") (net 21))
 (segment (start 91.81 67.47) (end 91.81 72.49) (width 0.2) (layer "F.Cu") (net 21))
 (segment (start 89.27 67.47) (end 89.27 72.49) (width 0.2) (layer "F.Cu") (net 22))
 (segment (start 89.27 72.49) (end 89.28 72.5) (width 0.2) (layer "F.Cu") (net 22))
 (segment (start 94.35 67.47) (end 94.35 72.49) (width 0.2) (layer "F.Cu") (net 20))
 (segment (start 94.35 72.49) (end 94.36 72.5) (width 0.2) (layer "F.Cu") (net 20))
 (segment (start 86.73 72.49) (end 86.74 72.5) (width 0.2) (layer "F.Cu") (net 23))
 (segment (start 86.73 67.47) (end 86.73 72.49) (width 0.2) (layer "F.Cu") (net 23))
 (segment (start 84.289 33.611) (end 79.11 38.79) (width 0.2) (layer "F.Cu") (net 13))
 (segment (start 79.11 72.49) (end 79.12 72.5) (width 0.2) (layer "F.Cu") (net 13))
 (segment (start 98.49 79.775) (end 101.03 79.775) (width 0.2) (layer "F.Cu") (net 13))
 (segment (start 97.8 74.8) (end 79.8 74.8) (width 0.2) (layer "F.Cu") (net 13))
 (segment (start 79.1 73.7) (end 79.12 73.68) (width 0.2) (layer "F.Cu") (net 13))
 (segment (start 112.7 74.75) (end 112.55 74.6) (width 0.2) (layer "F.Cu") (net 13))
 (segment (start 98.49 79.775) (end 98.49 75.49) (width 0.2) (layer "F.Cu") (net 13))
 (segment (start 98.49 75.49) (end 97.8 74.8) (width 0.2) (layer "F.Cu") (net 13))
 (segment (start 101 78.5) (end 101.03 78.53) (width 0.2) (layer "F.Cu") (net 13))
 (segment (start 112.4 74.75) (end 112.55 74.6) (width 0.2) (layer "F.Cu") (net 13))
 (segment (start 84.289 31.68) (end 84.289 33.611) (width 0.2) (layer "F.Cu") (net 13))
 (segment (start 101.03 78.53) (end 101.03 79.775) (width 0.2) (layer "F.Cu") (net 13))
 (segment (start 101 75.25) (end 101 78.5) (width 0.2) (layer "F.Cu") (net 13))
 (segment (start 79.11 67.47) (end 79.11 72.49) (width 0.2) (layer "F.Cu") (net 13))
 (segment (start 79.1 74.1) (end 79.1 73.7) (width 0.2) (layer "F.Cu") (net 13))
 (segment (start 101.5 74.75) (end 101 75.25) (width 0.2) (layer "F.Cu") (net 13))
 (segment (start 112.7 74.75) (end 110.16 74.75) (width 0.2) (layer "F.Cu") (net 13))
 (segment (start 118 72.75) (end 116 74.75) (width 0.2) (layer "F.Cu") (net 13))
 (segment (start 110.16 74.75) (end 112.4 74.75) (width 0.2) (layer "F.Cu") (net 13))
 (segment (start 110.16 74.75) (end 101.5 74.75) (width 0.2) (layer "F.Cu") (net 13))
 (segment (start 79.11 38.79) (end 79.11 67.47) (width 0.2) (layer "F.Cu") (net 13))
 (segment (start 116 74.75) (end 112.7 74.75) (width 0.2) (layer "F.Cu") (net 13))
 (segment (start 79.8 74.8) (end 79.1 74.1) (width 0.2) (layer "F.Cu") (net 13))
 (segment (start 112.55 74.6) (end 110.16 74.6) (width 0.2) (layer "F.Cu") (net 13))
 (segment (start 79.12 73.68) (end 79.12 72.9) (width 0.2) (layer "F.Cu") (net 13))
 (segment (start 86.68 42) (end 86.68 47.08) (width 0.2) (layer "F.Cu") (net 10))
 (segment (start 81.6 42) (end 81.6 47.08) (width 0.2) (layer "F.Cu") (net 12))
 (segment (start 76.57 67.47) (end 76.57 72.49) (width 0.2) (layer "F.Cu") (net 26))
 (segment (start 76.57 72.49) (end 76.58 72.5) (width 0.2) (layer "F.Cu") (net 26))
 (segment (start 76.57 39.83) (end 76.57 67.47) (width 0.2) (layer "F.Cu") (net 26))
 (segment (start 81.749 31.68) (end 81.749 34.651) (width 0.2) (layer "F.Cu") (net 26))
 (segment (start 81.749 34.651) (end 76.47 39.93) (width 0.2) (layer "F.Cu") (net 26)))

